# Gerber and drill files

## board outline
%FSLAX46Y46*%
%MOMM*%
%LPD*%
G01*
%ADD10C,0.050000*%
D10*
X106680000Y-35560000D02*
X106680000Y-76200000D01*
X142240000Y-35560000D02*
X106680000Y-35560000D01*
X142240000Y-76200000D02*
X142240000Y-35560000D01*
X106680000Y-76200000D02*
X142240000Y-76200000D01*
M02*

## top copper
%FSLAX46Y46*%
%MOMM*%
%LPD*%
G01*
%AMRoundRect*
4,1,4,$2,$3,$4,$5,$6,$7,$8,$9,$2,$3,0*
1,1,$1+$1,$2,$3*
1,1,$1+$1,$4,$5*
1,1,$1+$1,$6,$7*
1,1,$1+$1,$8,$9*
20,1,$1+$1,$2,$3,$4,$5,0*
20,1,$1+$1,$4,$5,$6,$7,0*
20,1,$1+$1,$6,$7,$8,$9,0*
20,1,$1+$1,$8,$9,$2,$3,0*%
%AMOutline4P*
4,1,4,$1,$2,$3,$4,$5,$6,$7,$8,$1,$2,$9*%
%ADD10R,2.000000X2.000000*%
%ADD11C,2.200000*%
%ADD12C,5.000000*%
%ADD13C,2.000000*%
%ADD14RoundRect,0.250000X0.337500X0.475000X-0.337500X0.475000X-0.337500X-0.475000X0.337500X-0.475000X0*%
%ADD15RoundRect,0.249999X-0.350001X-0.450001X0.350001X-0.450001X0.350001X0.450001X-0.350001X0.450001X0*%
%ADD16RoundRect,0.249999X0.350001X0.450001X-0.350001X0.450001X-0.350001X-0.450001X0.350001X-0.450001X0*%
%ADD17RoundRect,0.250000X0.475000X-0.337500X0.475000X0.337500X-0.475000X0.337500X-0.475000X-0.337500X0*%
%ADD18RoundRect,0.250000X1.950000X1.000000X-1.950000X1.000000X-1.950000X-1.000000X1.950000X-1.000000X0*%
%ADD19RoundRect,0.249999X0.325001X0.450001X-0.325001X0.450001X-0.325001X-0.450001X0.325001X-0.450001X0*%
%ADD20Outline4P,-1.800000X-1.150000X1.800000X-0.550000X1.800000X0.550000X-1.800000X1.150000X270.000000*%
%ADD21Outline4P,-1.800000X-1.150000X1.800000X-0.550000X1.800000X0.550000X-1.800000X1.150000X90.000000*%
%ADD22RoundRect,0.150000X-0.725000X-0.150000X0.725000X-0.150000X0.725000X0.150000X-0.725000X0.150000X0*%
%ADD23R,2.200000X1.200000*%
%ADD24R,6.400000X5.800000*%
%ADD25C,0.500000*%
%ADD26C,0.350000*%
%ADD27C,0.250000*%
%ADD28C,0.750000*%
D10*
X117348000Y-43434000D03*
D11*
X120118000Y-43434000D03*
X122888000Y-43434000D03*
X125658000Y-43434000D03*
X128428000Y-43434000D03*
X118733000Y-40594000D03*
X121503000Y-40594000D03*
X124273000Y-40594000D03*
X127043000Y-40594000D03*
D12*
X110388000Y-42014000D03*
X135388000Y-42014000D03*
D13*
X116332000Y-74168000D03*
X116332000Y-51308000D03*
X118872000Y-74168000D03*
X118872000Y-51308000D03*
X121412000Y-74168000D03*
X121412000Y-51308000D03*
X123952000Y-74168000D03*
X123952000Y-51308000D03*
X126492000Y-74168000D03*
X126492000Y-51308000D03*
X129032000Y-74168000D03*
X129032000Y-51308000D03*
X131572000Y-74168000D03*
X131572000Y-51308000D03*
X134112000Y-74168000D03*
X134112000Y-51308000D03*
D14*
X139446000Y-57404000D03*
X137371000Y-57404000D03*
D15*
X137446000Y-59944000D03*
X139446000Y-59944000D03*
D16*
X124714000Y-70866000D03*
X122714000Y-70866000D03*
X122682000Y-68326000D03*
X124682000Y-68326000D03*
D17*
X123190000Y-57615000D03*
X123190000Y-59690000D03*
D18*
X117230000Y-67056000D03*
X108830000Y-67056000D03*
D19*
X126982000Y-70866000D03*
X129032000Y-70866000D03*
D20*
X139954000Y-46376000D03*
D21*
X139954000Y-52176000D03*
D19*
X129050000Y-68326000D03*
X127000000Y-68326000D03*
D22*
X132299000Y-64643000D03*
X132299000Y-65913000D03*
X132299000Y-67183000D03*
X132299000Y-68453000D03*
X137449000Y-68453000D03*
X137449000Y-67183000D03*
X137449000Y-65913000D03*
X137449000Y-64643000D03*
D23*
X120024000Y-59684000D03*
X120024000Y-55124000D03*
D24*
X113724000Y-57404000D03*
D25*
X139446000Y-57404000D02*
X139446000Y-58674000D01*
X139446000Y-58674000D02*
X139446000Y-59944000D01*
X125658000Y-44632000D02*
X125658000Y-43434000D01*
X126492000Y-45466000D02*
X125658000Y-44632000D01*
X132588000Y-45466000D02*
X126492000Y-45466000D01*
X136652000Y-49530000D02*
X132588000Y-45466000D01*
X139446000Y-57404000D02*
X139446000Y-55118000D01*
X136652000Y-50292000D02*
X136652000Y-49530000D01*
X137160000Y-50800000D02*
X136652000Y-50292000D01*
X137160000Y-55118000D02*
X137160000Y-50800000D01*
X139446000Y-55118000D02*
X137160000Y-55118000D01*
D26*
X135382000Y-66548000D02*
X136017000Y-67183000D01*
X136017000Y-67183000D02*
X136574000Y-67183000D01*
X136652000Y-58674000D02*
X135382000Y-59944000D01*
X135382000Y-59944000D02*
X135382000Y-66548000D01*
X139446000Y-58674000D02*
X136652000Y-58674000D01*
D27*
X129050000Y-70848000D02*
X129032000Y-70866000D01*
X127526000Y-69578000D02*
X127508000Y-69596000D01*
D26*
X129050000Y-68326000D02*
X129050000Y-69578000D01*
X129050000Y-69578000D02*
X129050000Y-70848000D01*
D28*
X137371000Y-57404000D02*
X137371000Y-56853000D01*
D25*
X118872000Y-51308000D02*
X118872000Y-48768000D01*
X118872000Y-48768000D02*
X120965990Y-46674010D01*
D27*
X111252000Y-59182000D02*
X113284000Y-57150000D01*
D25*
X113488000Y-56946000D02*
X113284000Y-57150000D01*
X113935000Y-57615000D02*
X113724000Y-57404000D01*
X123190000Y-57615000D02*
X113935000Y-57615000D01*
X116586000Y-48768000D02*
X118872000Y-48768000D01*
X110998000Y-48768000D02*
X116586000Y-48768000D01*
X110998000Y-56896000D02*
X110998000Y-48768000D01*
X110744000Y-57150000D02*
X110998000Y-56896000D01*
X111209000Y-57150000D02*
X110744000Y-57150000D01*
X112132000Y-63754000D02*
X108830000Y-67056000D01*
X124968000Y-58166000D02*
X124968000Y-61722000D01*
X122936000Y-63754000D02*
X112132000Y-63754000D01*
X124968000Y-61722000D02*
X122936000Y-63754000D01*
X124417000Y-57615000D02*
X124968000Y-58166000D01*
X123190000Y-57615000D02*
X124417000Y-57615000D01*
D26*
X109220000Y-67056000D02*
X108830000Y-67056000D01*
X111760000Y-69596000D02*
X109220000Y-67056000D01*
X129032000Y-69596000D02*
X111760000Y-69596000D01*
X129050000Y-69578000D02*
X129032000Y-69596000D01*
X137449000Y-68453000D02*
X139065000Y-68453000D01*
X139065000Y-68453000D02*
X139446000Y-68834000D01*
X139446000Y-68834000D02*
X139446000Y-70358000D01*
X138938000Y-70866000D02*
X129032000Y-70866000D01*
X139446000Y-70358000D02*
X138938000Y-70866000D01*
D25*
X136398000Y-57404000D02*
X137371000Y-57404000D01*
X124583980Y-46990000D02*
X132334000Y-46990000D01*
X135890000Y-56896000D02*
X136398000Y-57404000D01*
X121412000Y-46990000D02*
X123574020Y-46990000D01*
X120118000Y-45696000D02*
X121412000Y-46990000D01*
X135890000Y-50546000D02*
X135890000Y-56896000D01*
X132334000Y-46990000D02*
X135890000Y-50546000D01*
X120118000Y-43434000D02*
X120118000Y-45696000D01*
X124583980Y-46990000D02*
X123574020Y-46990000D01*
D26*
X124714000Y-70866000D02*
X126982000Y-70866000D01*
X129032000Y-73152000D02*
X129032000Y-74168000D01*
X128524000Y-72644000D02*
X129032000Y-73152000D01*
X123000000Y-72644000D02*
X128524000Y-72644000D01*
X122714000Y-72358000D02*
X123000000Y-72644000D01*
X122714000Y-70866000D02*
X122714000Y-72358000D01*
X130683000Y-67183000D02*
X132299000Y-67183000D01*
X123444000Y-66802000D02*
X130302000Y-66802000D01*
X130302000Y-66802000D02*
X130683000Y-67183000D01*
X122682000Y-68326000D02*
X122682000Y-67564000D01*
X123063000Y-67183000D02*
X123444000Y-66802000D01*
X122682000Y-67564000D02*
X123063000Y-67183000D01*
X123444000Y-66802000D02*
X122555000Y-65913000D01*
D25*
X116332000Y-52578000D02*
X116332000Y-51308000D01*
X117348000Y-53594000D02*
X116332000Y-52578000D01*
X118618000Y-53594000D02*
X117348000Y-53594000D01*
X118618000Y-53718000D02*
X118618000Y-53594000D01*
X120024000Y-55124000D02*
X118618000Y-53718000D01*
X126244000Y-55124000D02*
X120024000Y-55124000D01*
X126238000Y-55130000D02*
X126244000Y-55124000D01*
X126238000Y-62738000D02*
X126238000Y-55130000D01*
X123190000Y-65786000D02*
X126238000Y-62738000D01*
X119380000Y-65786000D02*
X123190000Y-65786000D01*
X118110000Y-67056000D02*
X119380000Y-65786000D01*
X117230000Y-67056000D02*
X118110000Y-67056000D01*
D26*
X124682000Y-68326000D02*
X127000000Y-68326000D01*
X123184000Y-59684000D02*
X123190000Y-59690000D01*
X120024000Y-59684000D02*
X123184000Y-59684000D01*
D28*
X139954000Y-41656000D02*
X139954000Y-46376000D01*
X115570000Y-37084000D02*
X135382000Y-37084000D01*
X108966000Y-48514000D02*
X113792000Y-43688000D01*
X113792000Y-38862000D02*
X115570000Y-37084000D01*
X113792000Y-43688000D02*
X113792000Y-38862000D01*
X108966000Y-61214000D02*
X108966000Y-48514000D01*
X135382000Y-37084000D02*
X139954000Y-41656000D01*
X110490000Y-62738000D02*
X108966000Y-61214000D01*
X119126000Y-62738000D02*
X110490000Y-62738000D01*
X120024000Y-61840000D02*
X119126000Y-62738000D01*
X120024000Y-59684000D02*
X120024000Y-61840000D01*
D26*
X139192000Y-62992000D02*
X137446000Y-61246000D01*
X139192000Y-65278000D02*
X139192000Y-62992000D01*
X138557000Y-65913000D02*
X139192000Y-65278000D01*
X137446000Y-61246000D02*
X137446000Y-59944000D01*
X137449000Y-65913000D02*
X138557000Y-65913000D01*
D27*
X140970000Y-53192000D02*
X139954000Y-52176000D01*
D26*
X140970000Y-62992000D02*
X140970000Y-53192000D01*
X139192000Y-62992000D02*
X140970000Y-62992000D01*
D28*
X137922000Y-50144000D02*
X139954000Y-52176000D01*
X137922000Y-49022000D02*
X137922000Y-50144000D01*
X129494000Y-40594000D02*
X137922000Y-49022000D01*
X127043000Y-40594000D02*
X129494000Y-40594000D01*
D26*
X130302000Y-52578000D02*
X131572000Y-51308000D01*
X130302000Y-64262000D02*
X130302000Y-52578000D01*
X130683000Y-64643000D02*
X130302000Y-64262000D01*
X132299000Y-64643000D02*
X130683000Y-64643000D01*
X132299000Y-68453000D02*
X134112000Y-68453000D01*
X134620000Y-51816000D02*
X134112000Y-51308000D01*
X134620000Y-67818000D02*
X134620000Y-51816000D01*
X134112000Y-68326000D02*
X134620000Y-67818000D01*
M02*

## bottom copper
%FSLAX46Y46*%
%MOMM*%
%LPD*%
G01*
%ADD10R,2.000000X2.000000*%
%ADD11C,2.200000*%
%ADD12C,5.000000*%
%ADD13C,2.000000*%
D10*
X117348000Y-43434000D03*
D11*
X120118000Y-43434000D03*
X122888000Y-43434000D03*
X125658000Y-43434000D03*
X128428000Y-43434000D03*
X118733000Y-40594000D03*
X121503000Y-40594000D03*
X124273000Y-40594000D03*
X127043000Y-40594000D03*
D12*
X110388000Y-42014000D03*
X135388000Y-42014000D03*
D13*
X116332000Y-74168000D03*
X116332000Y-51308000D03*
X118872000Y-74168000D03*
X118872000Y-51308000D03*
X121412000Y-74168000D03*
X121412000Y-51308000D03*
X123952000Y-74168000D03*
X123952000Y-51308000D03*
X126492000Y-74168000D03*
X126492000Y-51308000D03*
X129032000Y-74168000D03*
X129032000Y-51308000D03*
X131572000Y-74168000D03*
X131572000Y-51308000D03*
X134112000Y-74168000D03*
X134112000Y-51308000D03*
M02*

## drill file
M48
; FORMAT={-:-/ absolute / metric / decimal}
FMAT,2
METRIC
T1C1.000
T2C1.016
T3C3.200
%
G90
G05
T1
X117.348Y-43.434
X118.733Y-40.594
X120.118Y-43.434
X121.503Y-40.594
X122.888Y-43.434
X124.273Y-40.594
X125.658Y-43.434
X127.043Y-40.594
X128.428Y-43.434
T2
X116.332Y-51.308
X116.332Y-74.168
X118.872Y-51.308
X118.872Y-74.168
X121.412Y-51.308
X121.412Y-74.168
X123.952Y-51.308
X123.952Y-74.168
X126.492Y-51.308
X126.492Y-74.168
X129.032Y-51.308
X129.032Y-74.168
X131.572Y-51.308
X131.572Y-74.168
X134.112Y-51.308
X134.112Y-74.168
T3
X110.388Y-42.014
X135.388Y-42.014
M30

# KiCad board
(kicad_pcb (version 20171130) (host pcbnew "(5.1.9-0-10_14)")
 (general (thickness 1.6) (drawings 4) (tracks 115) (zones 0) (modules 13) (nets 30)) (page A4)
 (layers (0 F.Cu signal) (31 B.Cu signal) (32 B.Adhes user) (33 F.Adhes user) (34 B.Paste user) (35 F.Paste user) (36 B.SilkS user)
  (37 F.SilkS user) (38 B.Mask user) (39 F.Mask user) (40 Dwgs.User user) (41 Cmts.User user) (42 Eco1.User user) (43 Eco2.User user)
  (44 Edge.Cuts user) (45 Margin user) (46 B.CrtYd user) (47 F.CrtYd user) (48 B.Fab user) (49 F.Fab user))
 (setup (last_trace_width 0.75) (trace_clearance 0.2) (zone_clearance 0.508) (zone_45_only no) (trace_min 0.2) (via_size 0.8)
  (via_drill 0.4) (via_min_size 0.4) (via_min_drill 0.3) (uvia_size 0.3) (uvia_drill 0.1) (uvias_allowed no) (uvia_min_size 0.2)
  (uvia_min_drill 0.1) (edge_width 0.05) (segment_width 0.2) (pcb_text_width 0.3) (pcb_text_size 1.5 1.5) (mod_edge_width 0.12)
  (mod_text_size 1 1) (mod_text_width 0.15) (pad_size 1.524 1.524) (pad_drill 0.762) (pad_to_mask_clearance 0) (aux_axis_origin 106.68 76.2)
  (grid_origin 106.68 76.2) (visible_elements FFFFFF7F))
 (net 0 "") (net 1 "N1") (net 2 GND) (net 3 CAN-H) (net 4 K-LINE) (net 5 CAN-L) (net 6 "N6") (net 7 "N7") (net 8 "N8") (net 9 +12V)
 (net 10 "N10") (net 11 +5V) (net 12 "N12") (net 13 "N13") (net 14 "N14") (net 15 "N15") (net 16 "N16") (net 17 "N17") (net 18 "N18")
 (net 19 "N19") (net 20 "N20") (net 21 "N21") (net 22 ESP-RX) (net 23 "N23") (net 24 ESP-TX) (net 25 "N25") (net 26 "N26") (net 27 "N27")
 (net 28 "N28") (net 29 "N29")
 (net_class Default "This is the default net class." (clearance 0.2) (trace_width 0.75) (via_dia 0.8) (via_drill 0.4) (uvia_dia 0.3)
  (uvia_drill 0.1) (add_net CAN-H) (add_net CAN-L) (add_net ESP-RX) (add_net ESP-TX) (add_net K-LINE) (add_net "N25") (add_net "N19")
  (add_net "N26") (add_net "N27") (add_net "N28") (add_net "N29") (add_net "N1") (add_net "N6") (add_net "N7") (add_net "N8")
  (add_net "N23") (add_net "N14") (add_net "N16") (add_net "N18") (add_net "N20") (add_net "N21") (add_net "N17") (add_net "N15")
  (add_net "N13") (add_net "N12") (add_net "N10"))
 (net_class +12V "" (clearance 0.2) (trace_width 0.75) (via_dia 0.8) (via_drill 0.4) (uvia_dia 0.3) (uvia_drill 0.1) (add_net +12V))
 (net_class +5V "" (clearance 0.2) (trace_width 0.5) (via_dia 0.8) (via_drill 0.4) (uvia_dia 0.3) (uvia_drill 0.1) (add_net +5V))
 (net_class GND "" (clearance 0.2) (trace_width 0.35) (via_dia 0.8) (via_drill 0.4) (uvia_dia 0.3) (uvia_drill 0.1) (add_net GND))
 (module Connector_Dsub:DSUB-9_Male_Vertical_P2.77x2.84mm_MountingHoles (layer B.Cu) (at 117.348 43.434)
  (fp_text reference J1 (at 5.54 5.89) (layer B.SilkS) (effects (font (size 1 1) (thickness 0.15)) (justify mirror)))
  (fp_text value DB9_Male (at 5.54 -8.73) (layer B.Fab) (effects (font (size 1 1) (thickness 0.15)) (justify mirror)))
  (pad 1 thru_hole rect (at 0 0) (size 2 2) (drill 1) (layers *.Cu *.Mask) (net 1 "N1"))
  (pad 2 thru_hole circle (at 2.77 0) (size 2.2 2.2) (drill 1) (layers *.Cu *.Mask) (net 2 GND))
  (pad 3 thru_hole circle (at 5.54 0) (size 2.2 2.2) (drill 1) (layers *.Cu *.Mask) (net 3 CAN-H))
  (pad 4 thru_hole circle (at 8.31 0) (size 2.2 2.2) (drill 1) (layers *.Cu *.Mask) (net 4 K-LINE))
  (pad 5 thru_hole circle (at 11.08 0) (size 2.2 2.2) (drill 1) (layers *.Cu *.Mask) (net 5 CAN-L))
  (pad 6 thru_hole circle (at 1.385 -2.84) (size 2.2 2.2) (drill 1) (layers *.Cu *.Mask) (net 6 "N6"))
  (pad 7 thru_hole circle (at 4.155 -2.84) (size 2.2 2.2) (drill 1) (layers *.Cu *.Mask) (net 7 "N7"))
  (pad 8 thru_hole circle (at 6.925 -2.84) (size 2.2 2.2) (drill 1) (layers *.Cu *.Mask) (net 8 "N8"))
  (pad 9 thru_hole circle (at 9.695 -2.84) (size 2.2 2.2) (drill 1) (layers *.Cu *.Mask) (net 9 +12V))
  (pad 0 thru_hole circle (at -6.96 -1.42) (size 5 5) (drill 3.2) (layers *.Cu *.Mask))
  (pad 0 thru_hole circle (at 18.04 -1.42) (size 5 5) (drill 3.2) (layers *.Cu *.Mask)))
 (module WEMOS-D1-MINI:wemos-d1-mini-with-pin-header (layer B.Cu) (at 125.222 62.738)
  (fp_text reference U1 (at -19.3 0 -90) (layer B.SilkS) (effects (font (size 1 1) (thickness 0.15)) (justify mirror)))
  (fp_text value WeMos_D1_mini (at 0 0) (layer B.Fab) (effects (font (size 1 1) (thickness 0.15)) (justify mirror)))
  (pad 8 thru_hole circle (at -8.89 11.43) (size 2 2) (drill 1.016) (layers *.Cu *.Mask) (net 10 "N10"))
  (pad 9 thru_hole circle (at -8.89 -11.43) (size 2 2) (drill 1.016) (layers *.Cu *.Mask) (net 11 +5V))
  (pad 7 thru_hole circle (at -6.35 11.43) (size 2 2) (drill 1.016) (layers *.Cu *.Mask) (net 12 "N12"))
  (pad 10 thru_hole circle (at -6.35 -11.43) (size 2 2) (drill 1.016) (layers *.Cu *.Mask) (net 2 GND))
  (pad 6 thru_hole circle (at -3.81 11.43) (size 2 2) (drill 1.016) (layers *.Cu *.Mask) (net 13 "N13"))
  (pad 11 thru_hole circle (at -3.81 -11.43) (size 2 2) (drill 1.016) (layers *.Cu *.Mask) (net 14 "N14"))
  (pad 5 thru_hole circle (at -1.27 11.43) (size 2 2) (drill 1.016) (layers *.Cu *.Mask) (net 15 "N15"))
  (pad 12 thru_hole circle (at -1.27 -11.43) (size 2 2) (drill 1.016) (layers *.Cu *.Mask) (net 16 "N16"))
  (pad 4 thru_hole circle (at 1.27 11.43) (size 2 2) (drill 1.016) (layers *.Cu *.Mask) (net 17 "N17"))
  (pad 13 thru_hole circle (at 1.27 -11.43) (size 2 2) (drill 1.016) (layers *.Cu *.Mask) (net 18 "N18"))
  (pad 3 thru_hole circle (at 3.81 11.43) (size 2 2) (drill 1.016) (layers *.Cu *.Mask) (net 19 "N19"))
  (pad 14 thru_hole circle (at 3.81 -11.43) (size 2 2) (drill 1.016) (layers *.Cu *.Mask) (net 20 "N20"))
  (pad 2 thru_hole circle (at 6.35 11.43) (size 2 2) (drill 1.016) (layers *.Cu *.Mask) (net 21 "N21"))
  (pad 15 thru_hole circle (at 6.35 -11.43) (size 2 2) (drill 1.016) (layers *.Cu *.Mask) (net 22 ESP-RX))
  (pad 1 thru_hole circle (at 8.89 11.43) (size 2 2) (drill 1.016) (layers *.Cu *.Mask) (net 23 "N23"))
  (pad 16 thru_hole circle (at 8.89 -11.43) (size 2 2) (drill 1.016) (layers *.Cu *.Mask) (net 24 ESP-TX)))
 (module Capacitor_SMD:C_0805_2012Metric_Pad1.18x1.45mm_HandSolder (layer F.Cu) (at 138.4085 57.404 180)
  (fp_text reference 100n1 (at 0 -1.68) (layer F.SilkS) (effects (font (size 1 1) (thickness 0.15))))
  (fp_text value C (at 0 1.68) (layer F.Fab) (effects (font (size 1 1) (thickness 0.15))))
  (pad 1 smd roundrect (at -1.0375 0 180) (size 1.175 1.45) (layers F.Cu F.Paste F.Mask) (roundrect_rratio 0.2127659574468085)
   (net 4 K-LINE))
  (pad 2 smd roundrect (at 1.0375 0 180) (size 1.175 1.45) (layers F.Cu F.Paste F.Mask) (roundrect_rratio 0.2127659574468085) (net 2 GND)))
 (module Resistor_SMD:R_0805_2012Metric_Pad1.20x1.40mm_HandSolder (layer F.Cu) (at 138.446 59.944)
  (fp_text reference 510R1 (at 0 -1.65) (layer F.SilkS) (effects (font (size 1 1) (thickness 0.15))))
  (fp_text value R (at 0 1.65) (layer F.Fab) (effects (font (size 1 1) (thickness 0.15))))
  (pad 1 smd roundrect (at -1 0) (size 1.2 1.4) (layers F.Cu F.Paste F.Mask) (roundrect_rratio 0.2083325) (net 9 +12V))
  (pad 2 smd roundrect (at 1 0) (size 1.2 1.4) (layers F.Cu F.Paste F.Mask) (roundrect_rratio 0.2083325) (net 4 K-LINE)))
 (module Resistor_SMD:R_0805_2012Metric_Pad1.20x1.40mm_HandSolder (layer F.Cu) (at 123.714 70.866 180)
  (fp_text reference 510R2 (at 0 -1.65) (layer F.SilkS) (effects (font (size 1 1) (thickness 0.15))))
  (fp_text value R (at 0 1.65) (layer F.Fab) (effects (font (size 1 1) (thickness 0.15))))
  (pad 1 smd roundrect (at -1 0 180) (size 1.2 1.4) (layers F.Cu F.Paste F.Mask) (roundrect_rratio 0.2083325) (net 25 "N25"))
  (pad 2 smd roundrect (at 1 0 180) (size 1.2 1.4) (layers F.Cu F.Paste F.Mask) (roundrect_rratio 0.2083325) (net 19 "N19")))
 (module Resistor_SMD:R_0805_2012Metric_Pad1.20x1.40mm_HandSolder (layer F.Cu) (at 123.682 68.326 180)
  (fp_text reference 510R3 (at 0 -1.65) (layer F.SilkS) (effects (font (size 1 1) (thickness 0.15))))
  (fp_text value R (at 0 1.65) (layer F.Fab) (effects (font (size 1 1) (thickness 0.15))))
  (pad 2 smd roundrect (at 1 0 180) (size 1.2 1.4) (layers F.Cu F.Paste F.Mask) (roundrect_rratio 0.2083325) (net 11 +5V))
  (pad 1 smd roundrect (at -1 0 180) (size 1.2 1.4) (layers F.Cu F.Paste F.Mask) (roundrect_rratio 0.2083325) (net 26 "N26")))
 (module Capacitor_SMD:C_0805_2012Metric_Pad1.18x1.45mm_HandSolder (layer F.Cu) (at 123.19 58.6525 90)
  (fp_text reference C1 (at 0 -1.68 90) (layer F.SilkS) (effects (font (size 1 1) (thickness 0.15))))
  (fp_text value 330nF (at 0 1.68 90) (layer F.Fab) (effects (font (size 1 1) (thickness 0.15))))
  (pad 2 smd roundrect (at 1.0375 0 90) (size 1.175 1.45) (layers F.Cu F.Paste F.Mask) (roundrect_rratio 0.2127659574468085) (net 2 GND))
  (pad 1 smd roundrect (at -1.0375 0 90) (size 1.175 1.45) (layers F.Cu F.Paste F.Mask) (roundrect_rratio 0.2127659574468085) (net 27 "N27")))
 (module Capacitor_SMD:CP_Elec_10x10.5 (layer F.Cu) (at 113.03 67.056 180)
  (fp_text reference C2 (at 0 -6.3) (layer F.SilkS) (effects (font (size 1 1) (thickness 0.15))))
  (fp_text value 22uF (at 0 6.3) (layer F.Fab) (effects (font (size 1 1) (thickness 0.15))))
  (pad 1 smd roundrect (at -4.2 0 180) (size 4.4 2.5) (layers F.Cu F.Paste F.Mask) (roundrect_rratio 0.1) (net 11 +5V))
  (pad 2 smd roundrect (at 4.2 0 180) (size 4.4 2.5) (layers F.Cu F.Paste F.Mask) (roundrect_rratio 0.1) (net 2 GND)))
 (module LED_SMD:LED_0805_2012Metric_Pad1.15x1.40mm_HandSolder (layer F.Cu) (at 128.007 70.866 180)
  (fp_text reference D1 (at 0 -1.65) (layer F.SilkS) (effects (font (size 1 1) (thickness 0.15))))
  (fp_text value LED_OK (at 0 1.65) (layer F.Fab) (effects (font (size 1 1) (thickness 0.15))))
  (pad 2 smd roundrect (at 1.025 0 180) (size 1.15 1.4) (layers F.Cu F.Paste F.Mask) (roundrect_rratio 0.2173904347826087) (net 25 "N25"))
  (pad 1 smd roundrect (at -1.025 0 180) (size 1.15 1.4) (layers F.Cu F.Paste F.Mask) (roundrect_rratio 0.2173904347826087) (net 2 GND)))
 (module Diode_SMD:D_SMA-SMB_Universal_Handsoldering (layer F.Cu) (at 139.954 49.276 270)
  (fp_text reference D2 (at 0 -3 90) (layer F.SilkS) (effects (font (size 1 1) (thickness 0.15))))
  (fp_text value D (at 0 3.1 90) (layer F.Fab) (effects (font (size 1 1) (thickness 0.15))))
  (pad 1 smd trapezoid (at -2.9 0 270) (size 3.6 1.7) (rect_delta 0.6 0) (layers F.Cu F.Paste F.Mask) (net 27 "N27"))
  (pad 2 smd trapezoid (at 2.9 0 90) (size 3.6 1.7) (rect_delta 0.6 0) (layers F.Cu F.Paste F.Mask) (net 9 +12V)))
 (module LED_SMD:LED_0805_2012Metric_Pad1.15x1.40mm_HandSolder (layer F.Cu) (at 128.025 68.326 180)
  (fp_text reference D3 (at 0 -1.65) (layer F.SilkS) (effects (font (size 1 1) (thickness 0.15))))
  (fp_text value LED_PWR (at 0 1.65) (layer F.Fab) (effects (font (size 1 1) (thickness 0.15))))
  (pad 1 smd roundrect (at -1.025 0 180) (size 1.15 1.4) (layers F.Cu F.Paste F.Mask) (roundrect_rratio 0.2173904347826087) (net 2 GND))
  (pad 2 smd roundrect (at 1.025 0 180) (size 1.15 1.4) (layers F.Cu F.Paste F.Mask) (roundrect_rratio 0.2173904347826087) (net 26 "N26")))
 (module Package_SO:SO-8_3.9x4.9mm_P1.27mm (layer F.Cu) (at 134.874 66.548)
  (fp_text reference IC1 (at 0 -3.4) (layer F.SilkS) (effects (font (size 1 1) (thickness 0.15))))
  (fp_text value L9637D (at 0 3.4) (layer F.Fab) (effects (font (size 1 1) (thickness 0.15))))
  (pad 1 smd roundrect (at -2.575 -1.905) (size 1.75 0.6) (layers F.Cu F.Paste F.Mask) (roundrect_rratio 0.25) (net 22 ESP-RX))
  (pad 2 smd roundrect (at -2.575 -0.635) (size 1.75 0.6) (layers F.Cu F.Paste F.Mask) (roundrect_rratio 0.25) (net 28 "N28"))
  (pad 3 smd roundrect (at -2.575 0.635) (size 1.75 0.6) (layers F.Cu F.Paste F.Mask) (roundrect_rratio 0.25) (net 11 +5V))
  (pad 4 smd roundrect (at -2.575 1.905) (size 1.75 0.6) (layers F.Cu F.Paste F.Mask) (roundrect_rratio 0.25) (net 24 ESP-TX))
  (pad 5 smd roundrect (at 2.575 1.905) (size 1.75 0.6) (layers F.Cu F.Paste F.Mask) (roundrect_rratio 0.25) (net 2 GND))
  (pad 6 smd roundrect (at 2.575 0.635) (size 1.75 0.6) (layers F.Cu F.Paste F.Mask) (roundrect_rratio 0.25) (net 4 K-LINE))
  (pad 7 smd roundrect (at 2.575 -0.635) (size 1.75 0.6) (layers F.Cu F.Paste F.Mask) (roundrect_rratio 0.25) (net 9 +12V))
  (pad 8 smd roundrect (at 2.575 -1.905) (size 1.75 0.6) (layers F.Cu F.Paste F.Mask) (roundrect_rratio 0.25) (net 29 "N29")))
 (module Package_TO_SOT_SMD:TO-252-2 (layer F.Cu) (at 115.824 57.404 180)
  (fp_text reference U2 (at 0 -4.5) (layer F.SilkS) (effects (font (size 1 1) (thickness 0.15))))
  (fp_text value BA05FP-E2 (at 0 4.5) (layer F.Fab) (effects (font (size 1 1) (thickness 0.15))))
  (pad 1 smd rect (at -4.2 -2.28 180) (size 2.2 1.2) (layers F.Cu F.Paste F.Mask) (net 27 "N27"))
  (pad 3 smd rect (at -4.2 2.28 180) (size 2.2 1.2) (layers F.Cu F.Paste F.Mask) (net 11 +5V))
  (pad 2 smd rect (at 2.1 0 180) (size 6.4 5.8) (layers F.Cu F.Mask) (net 2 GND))
  (pad "" smd rect (at 3.775 1.525 180) (size 3.05 2.75) (layers F.Paste))
  (pad "" smd rect (at 0.425 -1.525 180) (size 3.05 2.75) (layers F.Paste))
  (pad "" smd rect (at 3.775 -1.525 180) (size 3.05 2.75) (layers F.Paste))
  (pad "" smd rect (at 0.425 1.525 180) (size 3.05 2.75) (layers F.Paste)))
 (gr_line (start 106.68 35.56) (end 106.68 76.2) (layer Edge.Cuts) (width 0.05))
 (gr_line (start 142.24 35.56) (end 106.68 35.56) (layer Edge.Cuts) (width 0.05))
 (gr_line (start 142.24 76.2) (end 142.24 35.56) (layer Edge.Cuts) (width 0.05))
 (gr_line (start 106.68 76.2) (end 142.24 76.2) (layer Edge.Cuts) (width 0.05))
 (segment (start 139.446 57.404) (end 139.446 58.674) (width 0.5) (layer F.Cu) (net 4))
 (segment (start 139.446 58.674) (end 139.446 59.944) (width 0.5) (layer F.Cu) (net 4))
 (segment (start 125.658 44.632) (end 125.658 43.434) (width 0.5) (layer F.Cu) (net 4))
 (segment (start 126.492 45.466) (end 125.658 44.632) (width 0.5) (layer F.Cu) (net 4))
 (segment (start 132.588 45.466) (end 126.492 45.466) (width 0.5) (layer F.Cu) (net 4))
 (segment (start 136.652 49.53) (end 132.588 45.466) (width 0.5) (layer F.Cu) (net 4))
 (segment (start 139.446 57.404) (end 139.446 55.118) (width 0.5) (layer F.Cu) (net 4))
 (segment (start 136.652 50.292) (end 136.652 49.53) (width 0.5) (layer F.Cu) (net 4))
 (segment (start 137.16 50.8) (end 136.652 50.292) (width 0.5) (layer F.Cu) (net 4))
 (segment (start 137.16 55.118) (end 137.16 50.8) (width 0.5) (layer F.Cu) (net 4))
 (segment (start 139.446 55.118) (end 137.16 55.118) (width 0.5) (layer F.Cu) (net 4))
 (segment (start 135.382 66.548) (end 136.017 67.183) (width 0.35) (layer F.Cu) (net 4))
 (segment (start 136.017 67.183) (end 136.574 67.183) (width 0.35) (layer F.Cu) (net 4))
 (segment (start 136.652 58.674) (end 135.382 59.944) (width 0.35) (layer F.Cu) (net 4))
 (segment (start 135.382 59.944) (end 135.382 66.548) (width 0.35) (layer F.Cu) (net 4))
 (segment (start 139.446 58.674) (end 136.652 58.674) (width 0.35) (layer F.Cu) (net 4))
 (segment (start 129.05 70.848) (end 129.032 70.866) (width 0.25) (layer F.Cu) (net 2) (status 30))
 (segment (start 127.526 69.578) (end 127.508 69.596) (width 0.25) (layer F.Cu) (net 2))
 (segment (start 129.05 68.326) (end 129.05 69.578) (width 0.35) (layer F.Cu) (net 2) (status 10))
 (segment (start 129.05 69.578) (end 129.05 70.848) (width 0.35) (layer F.Cu) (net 2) (status 20))
 (segment (start 137.371 57.404) (end 137.371 56.853) (width 0.75) (layer F.Cu) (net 2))
 (segment (start 118.872 51.308) (end 118.872 48.768) (width 0.5) (layer F.Cu) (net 2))
 (segment (start 118.872 48.768) (end 120.96599 46.67401) (width 0.5) (layer F.Cu) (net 2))
 (segment (start 111.252 59.182) (end 113.284 57.15) (width 0.25) (layer F.Cu) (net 2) (status 20))
 (segment (start 113.488 56.946) (end 113.284 57.15) (width 0.5) (layer F.Cu) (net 2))
 (segment (start 113.935 57.615) (end 113.724 57.404) (width 0.5) (layer F.Cu) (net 2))
 (segment (start 123.19 57.615) (end 113.935 57.615) (width 0.5) (layer F.Cu) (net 2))
 (segment (start 116.586 48.768) (end 118.872 48.768) (width 0.5) (layer F.Cu) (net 2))
 (segment (start 110.998 48.768) (end 116.586 48.768) (width 0.5) (layer F.Cu) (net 2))
 (segment (start 110.998 56.896) (end 110.998 48.768) (width 0.5) (layer F.Cu) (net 2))
 (segment (start 110.744 57.15) (end 110.998 56.896) (width 0.5) (layer F.Cu) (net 2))
 (segment (start 111.209 57.15) (end 110.744 57.15) (width 0.5) (layer F.Cu) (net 2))
 (segment (start 112.132 63.754) (end 108.83 67.056) (width 0.5) (layer F.Cu) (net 2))
 (segment (start 124.968 58.166) (end 124.968 61.722) (width 0.5) (layer F.Cu) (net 2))
 (segment (start 122.936 63.754) (end 112.132 63.754) (width 0.5) (layer F.Cu) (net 2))
 (segment (start 124.968 61.722) (end 122.936 63.754) (width 0.5) (layer F.Cu) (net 2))
 (segment (start 124.417 57.615) (end 124.968 58.166) (width 0.5) (layer F.Cu) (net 2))
 (segment (start 123.19 57.615) (end 124.417 57.615) (width 0.5) (layer F.Cu) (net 2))
 (segment (start 109.22 67.056) (end 108.83 67.056) (width 0.35) (layer F.Cu) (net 2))
 (segment (start 111.76 69.596) (end 109.22 67.056) (width 0.35) (layer F.Cu) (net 2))
 (segment (start 129.032 69.596) (end 111.76 69.596) (width 0.35) (layer F.Cu) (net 2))
 (segment (start 129.05 69.578) (end 129.032 69.596) (width 0.35) (layer F.Cu) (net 2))
 (segment (start 137.449 68.453) (end 139.065 68.453) (width 0.35) (layer F.Cu) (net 2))
 (segment (start 139.065 68.453) (end 139.446 68.834) (width 0.35) (layer F.Cu) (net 2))
 (segment (start 139.446 68.834) (end 139.446 70.358) (width 0.35) (layer F.Cu) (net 2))
 (segment (start 138.938 70.866) (end 129.032 70.866) (width 0.35) (layer F.Cu) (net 2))
 (segment (start 139.446 70.358) (end 138.938 70.866) (width 0.35) (layer F.Cu) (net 2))
 (segment (start 136.398 57.404) (end 137.371 57.404) (width 0.5) (layer F.Cu) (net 2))
 (segment (start 124.58398 46.99) (end 132.334 46.99) (width 0.5) (layer F.Cu) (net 2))
 (segment (start 135.89 56.896) (end 136.398 57.404) (width 0.5) (layer F.Cu) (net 2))
 (segment (start 121.412 46.99) (end 123.57402 46.99) (width 0.5) (layer F.Cu) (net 2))
 (segment (start 120.118 45.696) (end 121.412 46.99) (width 0.5) (layer F.Cu) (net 2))
 (segment (start 135.89 50.546) (end 135.89 56.896) (width 0.5) (layer F.Cu) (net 2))
 (segment (start 132.334 46.99) (end 135.89 50.546) (width 0.5) (layer F.Cu) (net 2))
 (segment (start 120.118 43.434) (end 120.118 45.696) (width 0.5) (layer F.Cu) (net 2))
 (segment (start 124.58398 46.99) (end 123.57402 46.99) (width 0.5) (layer F.Cu) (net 2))
 (segment (start 124.714 70.866) (end 126.982 70.866) (width 0.35) (layer F.Cu) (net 25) (status 30))
 (segment (start 129.032 73.152) (end 129.032 74.168) (width 0.35) (layer F.Cu) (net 19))
 (segment (start 128.524 72.644) (end 129.032 73.152) (width 0.35) (layer F.Cu) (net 19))
 (segment (start 123 72.644) (end 128.524 72.644) (width 0.35) (layer F.Cu) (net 19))
 (segment (start 122.714 72.358) (end 123 72.644) (width 0.35) (layer F.Cu) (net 19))
 (segment (start 122.714 70.866) (end 122.714 72.358) (width 0.35) (layer F.Cu) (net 19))
 (segment (start 130.683 67.183) (end 132.299 67.183) (width 0.35) (layer F.Cu) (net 11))
 (segment (start 123.444 66.802) (end 130.302 66.802) (width 0.35) (layer F.Cu) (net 11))
 (segment (start 130.302 66.802) (end 130.683 67.183) (width 0.35) (layer F.Cu) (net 11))
 (segment (start 122.682 68.326) (end 122.682 67.564) (width 0.35) (layer F.Cu) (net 11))
 (segment (start 123.063 67.183) (end 123.444 66.802) (width 0.35) (layer F.Cu) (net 11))
 (segment (start 122.682 67.564) (end 123.063 67.183) (width 0.35) (layer F.Cu) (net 11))
 (segment (start 123.444 66.802) (end 122.555 65.913) (width 0.35) (layer F.Cu) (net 11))
 (segment (start 116.332 52.578) (end 116.332 51.308) (width 0.5) (layer F.Cu) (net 11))
 (segment (start 117.348 53.594) (end 116.332 52.578) (width 0.5) (layer F.Cu) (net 11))
 (segment (start 118.618 53.594) (end 117.348 53.594) (width 0.5) (layer F.Cu) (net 11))
 (segment (start 118.618 53.718) (end 118.618 53.594) (width 0.5) (layer F.Cu) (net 11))
 (segment (start 120.024 55.124) (end 118.618 53.718) (width 0.5) (layer F.Cu) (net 11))
 (segment (start 126.244 55.124) (end 120.024 55.124) (width 0.5) (layer F.Cu) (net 11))
 (segment (start 126.238 55.13) (end 126.244 55.124) (width 0.5) (layer F.Cu) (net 11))
 (segment (start 126.238 62.738) (end 126.238 55.13) (width 0.5) (layer F.Cu) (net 11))
 (segment (start 123.19 65.786) (end 126.238 62.738) (width 0.5) (layer F.Cu) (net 11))
 (segment (start 119.38 65.786) (end 123.19 65.786) (width 0.5) (layer F.Cu) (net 11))
 (segment (start 118.11 67.056) (end 119.38 65.786) (width 0.5) (layer F.Cu) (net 11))
 (segment (start 117.23 67.056) (end 118.11 67.056) (width 0.5) (layer F.Cu) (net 11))
 (segment (start 124.682 68.326) (end 127 68.326) (width 0.35) (layer F.Cu) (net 26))
 (segment (start 123.184 59.684) (end 123.19 59.69) (width 0.35) (layer F.Cu) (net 27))
 (segment (start 120.024 59.684) (end 123.184 59.684) (width 0.35) (layer F.Cu) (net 27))
 (segment (start 139.954 41.656) (end 139.954 46.376) (width 0.75) (layer F.Cu) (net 27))
 (segment (start 115.57 37.084) (end 135.382 37.084) (width 0.75) (layer F.Cu) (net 27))
 (segment (start 108.966 48.514) (end 113.792 43.688) (width 0.75) (layer F.Cu) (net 27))
 (segment (start 113.792 38.862) (end 115.57 37.084) (width 0.75) (layer F.Cu) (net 27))
 (segment (start 113.792 43.688) (end 113.792 38.862) (width 0.75) (layer F.Cu) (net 27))
 (segment (start 108.966 61.214) (end 108.966 48.514) (width 0.75) (layer F.Cu) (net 27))
 (segment (start 135.382 37.084) (end 139.954 41.656) (width 0.75) (layer F.Cu) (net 27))
 (segment (start 110.49 62.738) (end 108.966 61.214) (width 0.75) (layer F.Cu) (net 27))
 (segment (start 119.126 62.738) (end 110.49 62.738) (width 0.75) (layer F.Cu) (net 27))
 (segment (start 120.024 61.84) (end 119.126 62.738) (width 0.75) (layer F.Cu) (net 27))
 (segment (start 120.024 59.684) (end 120.024 61.84) (width 0.75) (layer F.Cu) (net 27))
 (segment (start 139.192 62.992) (end 137.446 61.246) (width 0.35) (layer F.Cu) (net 9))
 (segment (start 139.192 65.278) (end 139.192 62.992) (width 0.35) (layer F.Cu) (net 9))
 (segment (start 138.557 65.913) (end 139.192 65.278) (width 0.35) (layer F.Cu) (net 9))
 (segment (start 137.446 61.246) (end 137.446 59.944) (width 0.35) (layer F.Cu) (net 9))
 (segment (start 137.449 65.913) (end 138.557 65.913) (width 0.35) (layer F.Cu) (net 9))
 (segment (start 140.97 53.192) (end 139.954 52.176) (width 0.25) (layer F.Cu) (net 9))
 (segment (start 140.97 62.992) (end 140.97 53.192) (width 0.35) (layer F.Cu) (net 9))
 (segment (start 139.192 62.992) (end 140.97 62.992) (width 0.35) (layer F.Cu) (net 9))
 (segment (start 137.922 50.144) (end 139.954 52.176) (width 0.75) (layer F.Cu) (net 9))
 (segment (start 137.922 49.022) (end 137.922 50.144) (width 0.75) (layer F.Cu) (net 9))
 (segment (start 129.494 40.594) (end 137.922 49.022) (width 0.75) (layer F.Cu) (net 9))
 (segment (start 127.043 40.594) (end 129.494 40.594) (width 0.75) (layer F.Cu) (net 9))
 (segment (start 130.302 52.578) (end 131.572 51.308) (width 0.35) (layer F.Cu) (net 22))
 (segment (start 130.302 64.262) (end 130.302 52.578) (width 0.35) (layer F.Cu) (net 22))
 (segment (start 130.683 64.643) (end 130.302 64.262) (width 0.35) (layer F.Cu) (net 22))
 (segment (start 132.299 64.643) (end 130.683 64.643) (width 0.35) (layer F.Cu) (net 22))
 (segment (start 132.299 68.453) (end 134.112 68.453) (width 0.35) (layer F.Cu) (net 24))
 (segment (start 134.62 51.816) (end 134.112 51.308) (width 0.35) (layer F.Cu) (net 24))
 (segment (start 134.62 67.818) (end 134.62 51.816) (width 0.35) (layer F.Cu) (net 24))
 (segment (start 134.112 68.326) (end 134.62 67.818) (width 0.35) (layer F.Cu) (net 24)))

